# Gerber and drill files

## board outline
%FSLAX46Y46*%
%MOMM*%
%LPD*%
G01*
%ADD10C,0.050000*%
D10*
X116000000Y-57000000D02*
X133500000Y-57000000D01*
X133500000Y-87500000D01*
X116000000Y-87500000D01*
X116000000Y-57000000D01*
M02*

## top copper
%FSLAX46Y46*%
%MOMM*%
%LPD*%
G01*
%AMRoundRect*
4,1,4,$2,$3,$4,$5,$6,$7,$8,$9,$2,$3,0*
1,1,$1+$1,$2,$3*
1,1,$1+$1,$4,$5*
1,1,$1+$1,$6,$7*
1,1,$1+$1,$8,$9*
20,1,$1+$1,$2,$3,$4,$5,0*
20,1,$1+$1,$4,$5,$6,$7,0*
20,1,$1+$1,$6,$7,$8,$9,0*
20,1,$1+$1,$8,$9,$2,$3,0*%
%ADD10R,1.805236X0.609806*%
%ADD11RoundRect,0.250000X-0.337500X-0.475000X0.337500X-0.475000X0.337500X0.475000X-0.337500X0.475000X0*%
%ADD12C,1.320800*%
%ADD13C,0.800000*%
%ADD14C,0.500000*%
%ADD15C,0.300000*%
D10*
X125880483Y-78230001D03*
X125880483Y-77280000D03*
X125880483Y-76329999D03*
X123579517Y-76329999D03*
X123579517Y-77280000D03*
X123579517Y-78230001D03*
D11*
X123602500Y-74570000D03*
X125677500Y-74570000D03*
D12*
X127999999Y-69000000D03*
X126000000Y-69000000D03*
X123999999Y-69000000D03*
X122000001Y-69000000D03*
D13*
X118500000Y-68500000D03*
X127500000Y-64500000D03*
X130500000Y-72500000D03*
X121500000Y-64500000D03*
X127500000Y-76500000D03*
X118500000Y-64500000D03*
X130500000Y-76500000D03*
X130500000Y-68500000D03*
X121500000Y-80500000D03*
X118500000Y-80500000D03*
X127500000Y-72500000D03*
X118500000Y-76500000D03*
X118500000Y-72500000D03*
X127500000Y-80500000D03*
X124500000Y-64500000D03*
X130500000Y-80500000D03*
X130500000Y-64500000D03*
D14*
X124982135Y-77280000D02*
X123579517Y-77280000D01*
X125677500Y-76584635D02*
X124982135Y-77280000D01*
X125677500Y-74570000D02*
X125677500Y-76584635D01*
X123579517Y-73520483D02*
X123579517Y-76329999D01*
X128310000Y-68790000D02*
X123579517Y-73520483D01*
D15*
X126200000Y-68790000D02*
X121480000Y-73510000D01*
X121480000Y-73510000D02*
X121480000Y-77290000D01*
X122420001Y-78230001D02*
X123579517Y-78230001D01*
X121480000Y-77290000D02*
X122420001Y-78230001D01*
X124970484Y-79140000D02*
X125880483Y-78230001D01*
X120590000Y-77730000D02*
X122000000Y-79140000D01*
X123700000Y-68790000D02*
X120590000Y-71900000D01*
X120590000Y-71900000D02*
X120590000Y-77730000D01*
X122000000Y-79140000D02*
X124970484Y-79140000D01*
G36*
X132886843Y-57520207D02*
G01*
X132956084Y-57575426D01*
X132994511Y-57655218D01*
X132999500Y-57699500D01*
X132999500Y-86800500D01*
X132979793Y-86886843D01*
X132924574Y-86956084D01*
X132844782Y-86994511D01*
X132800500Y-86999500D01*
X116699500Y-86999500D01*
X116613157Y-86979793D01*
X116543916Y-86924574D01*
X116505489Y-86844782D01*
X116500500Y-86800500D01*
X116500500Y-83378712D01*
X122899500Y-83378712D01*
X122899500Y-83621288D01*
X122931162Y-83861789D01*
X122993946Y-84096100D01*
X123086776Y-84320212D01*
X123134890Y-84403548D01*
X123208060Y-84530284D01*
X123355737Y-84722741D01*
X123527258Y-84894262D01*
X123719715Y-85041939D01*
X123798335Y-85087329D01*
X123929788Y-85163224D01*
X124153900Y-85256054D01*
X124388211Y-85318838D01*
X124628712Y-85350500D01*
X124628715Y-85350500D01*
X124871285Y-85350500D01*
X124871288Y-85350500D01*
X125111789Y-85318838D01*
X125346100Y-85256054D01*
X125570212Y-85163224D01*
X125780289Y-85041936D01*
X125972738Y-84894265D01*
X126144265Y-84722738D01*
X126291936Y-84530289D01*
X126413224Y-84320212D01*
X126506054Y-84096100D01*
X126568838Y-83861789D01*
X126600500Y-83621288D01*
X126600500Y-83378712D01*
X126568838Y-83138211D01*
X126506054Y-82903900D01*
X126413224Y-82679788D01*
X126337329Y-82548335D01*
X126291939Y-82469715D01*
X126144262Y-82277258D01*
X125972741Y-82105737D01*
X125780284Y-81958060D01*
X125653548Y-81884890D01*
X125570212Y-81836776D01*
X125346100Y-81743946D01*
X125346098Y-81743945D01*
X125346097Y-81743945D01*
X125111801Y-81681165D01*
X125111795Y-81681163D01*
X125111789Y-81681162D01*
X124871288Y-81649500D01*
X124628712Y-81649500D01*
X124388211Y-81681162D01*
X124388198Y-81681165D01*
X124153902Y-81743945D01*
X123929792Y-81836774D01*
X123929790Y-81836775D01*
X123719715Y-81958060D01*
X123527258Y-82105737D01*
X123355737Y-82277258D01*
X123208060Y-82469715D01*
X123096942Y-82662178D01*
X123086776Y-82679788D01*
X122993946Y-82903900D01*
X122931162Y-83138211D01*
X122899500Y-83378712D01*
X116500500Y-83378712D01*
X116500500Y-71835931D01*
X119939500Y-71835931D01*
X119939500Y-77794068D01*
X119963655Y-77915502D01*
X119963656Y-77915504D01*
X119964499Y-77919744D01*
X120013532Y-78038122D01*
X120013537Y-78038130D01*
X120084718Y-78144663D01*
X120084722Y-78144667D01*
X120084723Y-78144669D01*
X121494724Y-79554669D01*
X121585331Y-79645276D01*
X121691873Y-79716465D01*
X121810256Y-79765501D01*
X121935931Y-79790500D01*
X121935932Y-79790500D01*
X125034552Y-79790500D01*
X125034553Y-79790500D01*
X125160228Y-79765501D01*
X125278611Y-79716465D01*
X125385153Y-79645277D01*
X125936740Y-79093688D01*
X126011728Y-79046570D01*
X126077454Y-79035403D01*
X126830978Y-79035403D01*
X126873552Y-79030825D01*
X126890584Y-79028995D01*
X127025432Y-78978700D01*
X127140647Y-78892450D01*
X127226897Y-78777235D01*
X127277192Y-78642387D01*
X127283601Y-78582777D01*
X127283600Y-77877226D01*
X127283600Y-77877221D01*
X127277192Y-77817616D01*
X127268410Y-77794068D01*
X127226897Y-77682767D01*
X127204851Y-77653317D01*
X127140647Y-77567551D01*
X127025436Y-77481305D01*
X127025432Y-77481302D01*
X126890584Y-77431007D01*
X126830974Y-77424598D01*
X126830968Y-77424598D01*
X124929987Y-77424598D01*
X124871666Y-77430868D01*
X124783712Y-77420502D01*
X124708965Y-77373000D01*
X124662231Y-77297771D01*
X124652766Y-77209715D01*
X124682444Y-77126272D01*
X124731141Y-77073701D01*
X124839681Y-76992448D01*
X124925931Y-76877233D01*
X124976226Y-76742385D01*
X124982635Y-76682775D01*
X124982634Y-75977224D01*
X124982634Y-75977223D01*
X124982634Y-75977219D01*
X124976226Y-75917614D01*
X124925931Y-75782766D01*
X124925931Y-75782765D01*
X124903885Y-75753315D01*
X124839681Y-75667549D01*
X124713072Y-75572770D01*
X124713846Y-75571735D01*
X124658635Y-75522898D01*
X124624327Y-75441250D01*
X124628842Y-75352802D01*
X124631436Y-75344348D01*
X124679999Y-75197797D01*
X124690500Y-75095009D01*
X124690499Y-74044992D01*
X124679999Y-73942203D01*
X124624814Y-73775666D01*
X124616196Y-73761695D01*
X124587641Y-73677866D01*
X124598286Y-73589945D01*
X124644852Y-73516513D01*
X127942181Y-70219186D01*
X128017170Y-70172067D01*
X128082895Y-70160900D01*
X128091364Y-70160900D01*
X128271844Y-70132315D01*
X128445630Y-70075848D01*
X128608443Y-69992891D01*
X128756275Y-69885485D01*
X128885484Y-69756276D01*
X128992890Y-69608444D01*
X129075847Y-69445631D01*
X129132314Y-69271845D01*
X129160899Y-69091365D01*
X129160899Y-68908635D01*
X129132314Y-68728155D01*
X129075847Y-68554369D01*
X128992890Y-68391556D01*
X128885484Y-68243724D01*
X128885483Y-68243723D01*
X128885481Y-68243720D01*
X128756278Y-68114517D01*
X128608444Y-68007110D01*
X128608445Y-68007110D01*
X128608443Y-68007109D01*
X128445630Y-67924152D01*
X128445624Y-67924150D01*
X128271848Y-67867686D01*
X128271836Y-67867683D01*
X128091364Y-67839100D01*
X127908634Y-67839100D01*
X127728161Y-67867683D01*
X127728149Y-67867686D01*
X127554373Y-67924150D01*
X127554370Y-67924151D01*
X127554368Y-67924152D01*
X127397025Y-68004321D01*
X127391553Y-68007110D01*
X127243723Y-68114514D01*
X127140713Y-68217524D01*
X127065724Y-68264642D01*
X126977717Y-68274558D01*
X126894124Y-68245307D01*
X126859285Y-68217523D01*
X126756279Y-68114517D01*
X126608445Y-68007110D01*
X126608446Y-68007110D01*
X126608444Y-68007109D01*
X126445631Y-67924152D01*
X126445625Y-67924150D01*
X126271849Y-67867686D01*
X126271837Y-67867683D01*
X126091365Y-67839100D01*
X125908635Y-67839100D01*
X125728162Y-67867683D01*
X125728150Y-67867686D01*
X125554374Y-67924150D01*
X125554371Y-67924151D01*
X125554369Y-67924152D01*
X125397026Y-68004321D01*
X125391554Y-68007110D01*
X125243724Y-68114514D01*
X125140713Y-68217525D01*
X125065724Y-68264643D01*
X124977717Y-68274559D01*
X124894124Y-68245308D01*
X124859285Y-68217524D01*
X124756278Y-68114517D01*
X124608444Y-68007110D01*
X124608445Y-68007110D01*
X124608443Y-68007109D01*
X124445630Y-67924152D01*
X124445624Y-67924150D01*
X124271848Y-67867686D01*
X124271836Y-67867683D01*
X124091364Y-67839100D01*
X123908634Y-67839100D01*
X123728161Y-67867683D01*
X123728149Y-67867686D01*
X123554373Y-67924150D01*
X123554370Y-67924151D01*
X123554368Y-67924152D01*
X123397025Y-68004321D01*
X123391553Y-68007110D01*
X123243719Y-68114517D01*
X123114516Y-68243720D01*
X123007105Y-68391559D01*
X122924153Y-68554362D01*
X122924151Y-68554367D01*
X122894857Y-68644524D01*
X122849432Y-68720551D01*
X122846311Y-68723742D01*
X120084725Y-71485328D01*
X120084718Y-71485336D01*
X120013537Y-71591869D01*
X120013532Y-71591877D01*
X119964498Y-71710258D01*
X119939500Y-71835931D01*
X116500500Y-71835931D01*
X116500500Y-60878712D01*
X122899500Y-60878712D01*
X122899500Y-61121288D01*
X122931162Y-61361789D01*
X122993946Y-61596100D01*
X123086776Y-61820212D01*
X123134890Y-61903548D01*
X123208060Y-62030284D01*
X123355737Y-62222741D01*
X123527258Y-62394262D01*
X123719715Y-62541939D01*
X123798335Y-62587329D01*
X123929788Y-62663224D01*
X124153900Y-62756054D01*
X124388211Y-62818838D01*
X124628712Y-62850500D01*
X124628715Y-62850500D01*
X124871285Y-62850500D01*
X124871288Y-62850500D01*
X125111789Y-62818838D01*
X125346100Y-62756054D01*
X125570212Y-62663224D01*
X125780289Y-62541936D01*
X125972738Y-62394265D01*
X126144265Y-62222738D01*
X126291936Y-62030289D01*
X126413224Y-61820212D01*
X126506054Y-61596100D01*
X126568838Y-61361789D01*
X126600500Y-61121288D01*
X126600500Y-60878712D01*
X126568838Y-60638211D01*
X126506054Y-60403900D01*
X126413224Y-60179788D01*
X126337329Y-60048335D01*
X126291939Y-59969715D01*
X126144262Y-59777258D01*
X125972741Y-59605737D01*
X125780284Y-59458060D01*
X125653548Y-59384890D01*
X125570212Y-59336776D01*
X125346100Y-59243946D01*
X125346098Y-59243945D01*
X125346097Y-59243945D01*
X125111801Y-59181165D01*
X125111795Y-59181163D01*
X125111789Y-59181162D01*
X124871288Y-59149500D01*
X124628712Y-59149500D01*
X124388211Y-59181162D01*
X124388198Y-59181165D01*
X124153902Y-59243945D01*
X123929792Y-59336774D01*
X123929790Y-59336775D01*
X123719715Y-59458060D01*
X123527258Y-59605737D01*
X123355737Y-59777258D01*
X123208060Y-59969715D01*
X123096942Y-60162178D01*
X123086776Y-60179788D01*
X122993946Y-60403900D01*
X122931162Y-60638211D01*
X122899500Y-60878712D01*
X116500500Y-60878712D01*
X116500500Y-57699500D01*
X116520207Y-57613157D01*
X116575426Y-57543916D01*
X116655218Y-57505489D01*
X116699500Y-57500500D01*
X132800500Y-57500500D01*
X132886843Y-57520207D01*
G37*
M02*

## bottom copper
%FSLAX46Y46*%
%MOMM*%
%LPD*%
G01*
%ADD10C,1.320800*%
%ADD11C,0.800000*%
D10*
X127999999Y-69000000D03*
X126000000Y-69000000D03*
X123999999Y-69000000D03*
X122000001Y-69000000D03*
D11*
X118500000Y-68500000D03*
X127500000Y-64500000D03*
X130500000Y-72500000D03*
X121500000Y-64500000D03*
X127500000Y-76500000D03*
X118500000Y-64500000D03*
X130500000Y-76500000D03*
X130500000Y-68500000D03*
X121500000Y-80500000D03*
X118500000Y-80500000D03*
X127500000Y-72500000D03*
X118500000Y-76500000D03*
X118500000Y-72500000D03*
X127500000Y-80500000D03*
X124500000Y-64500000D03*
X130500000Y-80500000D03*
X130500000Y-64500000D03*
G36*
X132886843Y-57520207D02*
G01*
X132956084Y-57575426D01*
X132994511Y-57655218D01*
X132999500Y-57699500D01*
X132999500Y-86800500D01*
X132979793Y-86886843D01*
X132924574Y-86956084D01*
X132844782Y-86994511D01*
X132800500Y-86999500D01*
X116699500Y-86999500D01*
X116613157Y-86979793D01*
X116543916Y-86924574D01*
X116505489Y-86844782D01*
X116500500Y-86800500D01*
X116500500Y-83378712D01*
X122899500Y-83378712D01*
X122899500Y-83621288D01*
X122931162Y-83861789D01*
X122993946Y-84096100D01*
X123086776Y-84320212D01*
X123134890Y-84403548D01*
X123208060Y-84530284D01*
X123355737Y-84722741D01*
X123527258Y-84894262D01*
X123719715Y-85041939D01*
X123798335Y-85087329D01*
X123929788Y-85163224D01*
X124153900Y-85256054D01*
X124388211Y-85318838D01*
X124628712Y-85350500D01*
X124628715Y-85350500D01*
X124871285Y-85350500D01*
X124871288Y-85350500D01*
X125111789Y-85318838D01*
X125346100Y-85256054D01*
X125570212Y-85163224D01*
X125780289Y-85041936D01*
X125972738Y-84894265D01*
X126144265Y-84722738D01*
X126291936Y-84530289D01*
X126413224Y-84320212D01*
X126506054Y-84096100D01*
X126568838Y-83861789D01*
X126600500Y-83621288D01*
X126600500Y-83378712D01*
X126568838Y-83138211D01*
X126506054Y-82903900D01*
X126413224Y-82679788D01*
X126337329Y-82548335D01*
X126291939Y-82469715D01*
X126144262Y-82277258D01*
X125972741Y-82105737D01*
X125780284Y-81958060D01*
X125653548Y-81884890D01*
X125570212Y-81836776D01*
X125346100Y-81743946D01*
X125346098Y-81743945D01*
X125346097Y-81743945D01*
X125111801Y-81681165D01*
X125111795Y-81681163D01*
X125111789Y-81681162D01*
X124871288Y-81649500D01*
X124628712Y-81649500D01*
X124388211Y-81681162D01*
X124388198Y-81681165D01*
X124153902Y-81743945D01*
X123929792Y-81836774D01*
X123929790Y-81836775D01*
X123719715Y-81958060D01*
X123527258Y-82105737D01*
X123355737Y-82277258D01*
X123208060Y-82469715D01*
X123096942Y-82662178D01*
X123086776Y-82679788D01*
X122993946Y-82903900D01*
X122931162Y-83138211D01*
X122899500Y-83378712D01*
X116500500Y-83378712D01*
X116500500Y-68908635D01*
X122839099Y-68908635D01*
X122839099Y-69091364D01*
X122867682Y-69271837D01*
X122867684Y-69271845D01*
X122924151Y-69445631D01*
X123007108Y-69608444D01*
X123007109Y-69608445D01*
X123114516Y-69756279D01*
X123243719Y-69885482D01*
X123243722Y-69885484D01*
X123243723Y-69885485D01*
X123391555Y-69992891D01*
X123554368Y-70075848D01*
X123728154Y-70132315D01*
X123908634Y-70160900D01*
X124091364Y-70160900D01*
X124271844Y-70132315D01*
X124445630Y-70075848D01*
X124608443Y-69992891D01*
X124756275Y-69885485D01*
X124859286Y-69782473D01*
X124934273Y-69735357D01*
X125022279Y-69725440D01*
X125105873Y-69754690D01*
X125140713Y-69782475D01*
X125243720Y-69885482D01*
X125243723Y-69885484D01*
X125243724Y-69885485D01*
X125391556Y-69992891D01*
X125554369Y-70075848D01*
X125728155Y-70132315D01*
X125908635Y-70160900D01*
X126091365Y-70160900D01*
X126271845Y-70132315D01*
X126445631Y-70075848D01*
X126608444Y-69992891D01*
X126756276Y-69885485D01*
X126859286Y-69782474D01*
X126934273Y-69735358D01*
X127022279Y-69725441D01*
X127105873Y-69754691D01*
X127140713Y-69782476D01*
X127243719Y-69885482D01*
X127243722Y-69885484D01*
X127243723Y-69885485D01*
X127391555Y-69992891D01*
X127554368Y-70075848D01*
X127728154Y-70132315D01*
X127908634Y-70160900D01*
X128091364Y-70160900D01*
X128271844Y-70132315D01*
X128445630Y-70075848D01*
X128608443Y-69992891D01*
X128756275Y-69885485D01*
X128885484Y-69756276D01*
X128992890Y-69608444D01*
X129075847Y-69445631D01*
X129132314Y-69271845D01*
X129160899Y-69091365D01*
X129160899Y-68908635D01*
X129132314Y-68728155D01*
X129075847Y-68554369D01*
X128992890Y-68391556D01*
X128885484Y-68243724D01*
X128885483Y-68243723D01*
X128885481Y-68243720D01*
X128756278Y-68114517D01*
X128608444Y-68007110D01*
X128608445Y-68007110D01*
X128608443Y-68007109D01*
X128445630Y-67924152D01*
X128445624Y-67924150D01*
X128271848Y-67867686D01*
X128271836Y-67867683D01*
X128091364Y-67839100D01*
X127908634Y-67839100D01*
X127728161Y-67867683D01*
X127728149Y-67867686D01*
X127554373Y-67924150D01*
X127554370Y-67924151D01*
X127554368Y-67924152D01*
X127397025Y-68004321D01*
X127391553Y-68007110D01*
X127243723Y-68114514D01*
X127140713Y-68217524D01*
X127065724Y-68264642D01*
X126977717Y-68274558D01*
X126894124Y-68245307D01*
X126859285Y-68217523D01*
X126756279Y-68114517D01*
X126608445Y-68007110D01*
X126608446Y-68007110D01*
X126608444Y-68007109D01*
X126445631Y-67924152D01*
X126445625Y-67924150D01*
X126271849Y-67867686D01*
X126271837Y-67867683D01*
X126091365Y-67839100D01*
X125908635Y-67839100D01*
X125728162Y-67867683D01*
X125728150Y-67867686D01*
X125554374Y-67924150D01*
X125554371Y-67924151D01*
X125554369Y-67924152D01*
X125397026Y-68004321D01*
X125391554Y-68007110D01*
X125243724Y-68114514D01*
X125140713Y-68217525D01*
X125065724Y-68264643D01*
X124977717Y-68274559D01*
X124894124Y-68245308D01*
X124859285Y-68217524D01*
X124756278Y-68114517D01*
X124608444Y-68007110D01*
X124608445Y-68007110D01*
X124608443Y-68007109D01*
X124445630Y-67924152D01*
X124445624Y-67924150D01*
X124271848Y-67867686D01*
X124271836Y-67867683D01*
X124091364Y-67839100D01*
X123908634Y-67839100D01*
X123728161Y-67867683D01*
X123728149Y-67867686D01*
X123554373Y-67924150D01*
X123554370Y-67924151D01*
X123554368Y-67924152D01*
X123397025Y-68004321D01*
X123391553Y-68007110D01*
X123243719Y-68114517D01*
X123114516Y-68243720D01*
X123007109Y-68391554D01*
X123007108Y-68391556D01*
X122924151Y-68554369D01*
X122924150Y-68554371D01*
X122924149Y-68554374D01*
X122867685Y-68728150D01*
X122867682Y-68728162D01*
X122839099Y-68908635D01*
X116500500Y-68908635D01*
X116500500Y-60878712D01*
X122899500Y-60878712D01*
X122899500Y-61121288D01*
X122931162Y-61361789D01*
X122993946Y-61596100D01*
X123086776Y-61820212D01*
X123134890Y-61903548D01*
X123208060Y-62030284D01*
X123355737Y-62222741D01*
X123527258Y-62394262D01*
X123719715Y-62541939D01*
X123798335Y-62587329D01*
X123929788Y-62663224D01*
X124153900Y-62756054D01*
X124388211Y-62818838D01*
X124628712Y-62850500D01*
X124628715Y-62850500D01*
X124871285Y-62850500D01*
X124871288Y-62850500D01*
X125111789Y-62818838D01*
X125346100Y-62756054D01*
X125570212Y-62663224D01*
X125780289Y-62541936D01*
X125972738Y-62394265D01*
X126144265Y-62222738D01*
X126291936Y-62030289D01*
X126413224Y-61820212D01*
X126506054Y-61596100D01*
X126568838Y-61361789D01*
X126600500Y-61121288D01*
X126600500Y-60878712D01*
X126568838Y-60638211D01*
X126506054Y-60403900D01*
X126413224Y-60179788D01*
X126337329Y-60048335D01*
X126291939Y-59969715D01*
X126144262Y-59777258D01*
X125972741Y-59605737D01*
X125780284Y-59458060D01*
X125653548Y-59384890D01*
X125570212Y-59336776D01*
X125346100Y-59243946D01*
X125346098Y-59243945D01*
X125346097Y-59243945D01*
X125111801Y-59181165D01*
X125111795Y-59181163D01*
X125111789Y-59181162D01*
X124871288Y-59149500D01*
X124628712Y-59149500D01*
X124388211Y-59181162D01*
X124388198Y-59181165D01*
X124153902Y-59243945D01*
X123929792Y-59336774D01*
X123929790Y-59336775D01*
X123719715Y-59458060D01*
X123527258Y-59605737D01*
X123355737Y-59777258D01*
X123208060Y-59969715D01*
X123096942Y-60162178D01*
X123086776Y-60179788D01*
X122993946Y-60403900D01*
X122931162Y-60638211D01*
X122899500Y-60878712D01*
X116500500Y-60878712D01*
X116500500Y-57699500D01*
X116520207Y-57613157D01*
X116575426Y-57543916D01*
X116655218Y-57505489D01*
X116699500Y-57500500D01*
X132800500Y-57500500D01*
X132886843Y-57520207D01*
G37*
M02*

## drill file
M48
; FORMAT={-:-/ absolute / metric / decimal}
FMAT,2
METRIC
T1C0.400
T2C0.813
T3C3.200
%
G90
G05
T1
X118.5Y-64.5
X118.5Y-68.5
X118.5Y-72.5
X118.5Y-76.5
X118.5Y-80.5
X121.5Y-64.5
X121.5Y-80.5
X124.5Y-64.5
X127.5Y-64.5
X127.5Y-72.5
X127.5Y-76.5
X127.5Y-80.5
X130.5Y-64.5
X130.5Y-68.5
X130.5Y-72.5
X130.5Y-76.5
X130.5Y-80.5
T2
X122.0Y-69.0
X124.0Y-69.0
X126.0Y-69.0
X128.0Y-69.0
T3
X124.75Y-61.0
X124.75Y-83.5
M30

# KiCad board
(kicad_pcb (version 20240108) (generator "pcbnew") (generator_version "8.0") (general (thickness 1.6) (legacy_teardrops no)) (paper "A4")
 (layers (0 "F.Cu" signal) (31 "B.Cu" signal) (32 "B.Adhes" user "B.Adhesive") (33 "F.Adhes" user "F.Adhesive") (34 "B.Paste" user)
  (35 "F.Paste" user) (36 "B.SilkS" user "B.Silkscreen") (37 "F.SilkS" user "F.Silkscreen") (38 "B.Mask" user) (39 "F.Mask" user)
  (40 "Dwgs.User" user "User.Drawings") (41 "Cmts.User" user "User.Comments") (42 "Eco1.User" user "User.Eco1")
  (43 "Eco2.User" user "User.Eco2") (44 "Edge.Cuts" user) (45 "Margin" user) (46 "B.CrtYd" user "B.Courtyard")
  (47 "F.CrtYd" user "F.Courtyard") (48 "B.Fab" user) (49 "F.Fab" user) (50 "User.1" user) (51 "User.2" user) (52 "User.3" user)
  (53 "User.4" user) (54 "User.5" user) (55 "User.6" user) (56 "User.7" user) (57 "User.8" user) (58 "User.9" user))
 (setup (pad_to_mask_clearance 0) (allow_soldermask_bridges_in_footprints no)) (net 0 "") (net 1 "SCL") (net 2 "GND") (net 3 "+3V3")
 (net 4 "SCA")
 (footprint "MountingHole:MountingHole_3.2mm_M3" (layer "F.Cu") (at 124.75 83.5)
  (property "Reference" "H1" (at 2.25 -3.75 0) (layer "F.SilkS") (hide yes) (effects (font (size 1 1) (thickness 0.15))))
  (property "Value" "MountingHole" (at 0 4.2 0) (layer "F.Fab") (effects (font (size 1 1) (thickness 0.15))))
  (pad "" np_thru_hole circle (at 0 0) (size 3.2 3.2) (drill 3.2) (layers "*.Cu" "*.Mask")))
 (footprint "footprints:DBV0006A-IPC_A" (layer "F.Cu") (at 124.73 77.28 180)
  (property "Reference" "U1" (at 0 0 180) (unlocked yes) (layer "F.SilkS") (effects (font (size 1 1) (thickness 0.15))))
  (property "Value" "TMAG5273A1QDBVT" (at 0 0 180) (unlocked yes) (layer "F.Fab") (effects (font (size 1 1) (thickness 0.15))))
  (pad "1" smd rect (at -1.150483 -0.950001 180) (size 1.805236 0.609806) (layers "F.Cu" "F.Paste" "F.Mask") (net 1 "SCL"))
  (pad "2" smd rect (at -1.150483 0 180) (size 1.805236 0.609806) (layers "F.Cu" "F.Paste" "F.Mask") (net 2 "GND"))
  (pad "3" smd rect (at -1.150483 0.950001 180) (size 1.805236 0.609806) (layers "F.Cu" "F.Paste" "F.Mask") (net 2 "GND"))
  (pad "4" smd rect (at 1.150483 0.950001 180) (size 1.805236 0.609806) (layers "F.Cu" "F.Paste" "F.Mask") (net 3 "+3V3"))
  (pad "5" smd rect (at 1.150483 0 180) (size 1.805236 0.609806) (layers "F.Cu" "F.Paste" "F.Mask") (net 2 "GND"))
  (pad "6" smd rect (at 1.150483 -0.950001 180) (size 1.805236 0.609806) (layers "F.Cu" "F.Paste" "F.Mask") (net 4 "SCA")))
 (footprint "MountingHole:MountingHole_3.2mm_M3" (layer "F.Cu") (at 124.75 61)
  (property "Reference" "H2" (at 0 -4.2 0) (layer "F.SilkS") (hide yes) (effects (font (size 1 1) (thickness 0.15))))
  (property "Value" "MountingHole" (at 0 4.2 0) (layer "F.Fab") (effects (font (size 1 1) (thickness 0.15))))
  (pad "" np_thru_hole circle (at 0 0) (size 3.2 3.2) (drill 3.2) (layers "*.Cu" "*.Mask")))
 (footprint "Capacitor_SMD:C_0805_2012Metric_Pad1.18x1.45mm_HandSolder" (layer "F.Cu") (at 124.64 74.57)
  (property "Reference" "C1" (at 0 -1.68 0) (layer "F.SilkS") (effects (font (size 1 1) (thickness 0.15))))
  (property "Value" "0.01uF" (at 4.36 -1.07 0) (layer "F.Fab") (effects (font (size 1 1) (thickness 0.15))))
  (pad "1" smd roundrect (at -1.0375 0) (size 1.175 1.45) (layers "F.Cu" "F.Paste" "F.Mask") (roundrect_rratio 0.212766) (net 3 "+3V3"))
  (pad "2" smd roundrect (at 1.0375 0) (size 1.175 1.45) (layers "F.Cu" "F.Paste" "F.Mask") (roundrect_rratio 0.212766) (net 2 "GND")))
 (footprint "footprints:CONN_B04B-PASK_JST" (layer "B.Cu") (at 127.999999 69 180)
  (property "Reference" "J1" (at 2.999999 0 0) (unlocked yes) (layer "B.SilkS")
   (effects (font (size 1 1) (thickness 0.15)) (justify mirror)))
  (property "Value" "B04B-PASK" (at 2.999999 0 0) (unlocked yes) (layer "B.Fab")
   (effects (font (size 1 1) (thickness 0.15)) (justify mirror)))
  (pad "1" thru_hole circle (at 0 0 180) (size 1.3208 1.3208) (drill 0.8128) (layers "*.Cu" "*.Mask") (remove_unused_layers no)
   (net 3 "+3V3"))
  (pad "2" thru_hole circle (at 1.999999 0 180) (size 1.3208 1.3208) (drill 0.8128) (layers "*.Cu" "*.Mask") (remove_unused_layers no)
   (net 1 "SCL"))
  (pad "3" thru_hole circle (at 4 0 180) (size 1.3208 1.3208) (drill 0.8128) (layers "*.Cu" "*.Mask") (remove_unused_layers no)
   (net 4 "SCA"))
  (pad "4" thru_hole circle (at 5.999998 0 180) (size 1.3208 1.3208) (drill 0.8128) (layers "*.Cu" "*.Mask") (remove_unused_layers no)
   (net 2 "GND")))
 (gr_rect (start 116 57) (end 133.5 87.5) (stroke (width 0.05) (type default)) (fill none) (layer "Edge.Cuts"))
 (segment (start 124.982135 77.28) (end 123.579517 77.28) (width 0.5) (layer "F.Cu") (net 2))
 (segment (start 125.6775 76.584635) (end 124.982135 77.28) (width 0.5) (layer "F.Cu") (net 2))
 (segment (start 125.6775 74.57) (end 125.6775 76.584635) (width 0.5) (layer "F.Cu") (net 2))
 (via (at 118.5 68.5) (size 0.8) (drill 0.4) (layers "F.Cu" "B.Cu") (free yes) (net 2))
 (via (at 127.5 64.5) (size 0.8) (drill 0.4) (layers "F.Cu" "B.Cu") (free yes) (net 2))
 (via (at 130.5 72.5) (size 0.8) (drill 0.4) (layers "F.Cu" "B.Cu") (free yes) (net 2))
 (via (at 121.5 64.5) (size 0.8) (drill 0.4) (layers "F.Cu" "B.Cu") (free yes) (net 2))
 (via (at 127.5 76.5) (size 0.8) (drill 0.4) (layers "F.Cu" "B.Cu") (free yes) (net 2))
 (via (at 118.5 64.5) (size 0.8) (drill 0.4) (layers "F.Cu" "B.Cu") (free yes) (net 2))
 (via (at 130.5 76.5) (size 0.8) (drill 0.4) (layers "F.Cu" "B.Cu") (free yes) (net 2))
 (via (at 130.5 68.5) (size 0.8) (drill 0.4) (layers "F.Cu" "B.Cu") (free yes) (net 2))
 (via (at 121.5 80.5) (size 0.8) (drill 0.4) (layers "F.Cu" "B.Cu") (free yes) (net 2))
 (via (at 118.5 80.5) (size 0.8) (drill 0.4) (layers "F.Cu" "B.Cu") (free yes) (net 2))
 (via (at 127.5 72.5) (size 0.8) (drill 0.4) (layers "F.Cu" "B.Cu") (free yes) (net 2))
 (via (at 118.5 76.5) (size 0.8) (drill 0.4) (layers "F.Cu" "B.Cu") (free yes) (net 2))
 (via (at 118.5 72.5) (size 0.8) (drill 0.4) (layers "F.Cu" "B.Cu") (free yes) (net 2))
 (via (at 127.5 80.5) (size 0.8) (drill 0.4) (layers "F.Cu" "B.Cu") (free yes) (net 2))
 (via (at 124.5 64.5) (size 0.8) (drill 0.4) (layers "F.Cu" "B.Cu") (free yes) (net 2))
 (via (at 130.5 80.5) (size 0.8) (drill 0.4) (layers "F.Cu" "B.Cu") (free yes) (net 2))
 (via (at 130.5 64.5) (size 0.8) (drill 0.4) (layers "F.Cu" "B.Cu") (free yes) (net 2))
 (segment (start 123.579517 73.520483) (end 123.579517 76.329999) (width 0.5) (layer "F.Cu") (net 3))
 (segment (start 128.31 68.79) (end 123.579517 73.520483) (width 0.5) (layer "F.Cu") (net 3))
 (segment (start 126.2 68.79) (end 121.48 73.51) (width 0.3) (layer "F.Cu") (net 1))
 (segment (start 121.48 73.51) (end 121.48 77.29) (width 0.3) (layer "F.Cu") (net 1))
 (segment (start 122.420001 78.230001) (end 123.579517 78.230001) (width 0.3) (layer "F.Cu") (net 1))
 (segment (start 121.48 77.29) (end 122.420001 78.230001) (width 0.3) (layer "F.Cu") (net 1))
 (segment (start 124.970484 79.14) (end 125.880483 78.230001) (width 0.3) (layer "F.Cu") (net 4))
 (segment (start 120.59 77.73) (end 122 79.14) (width 0.3) (layer "F.Cu") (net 4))
 (segment (start 123.7 68.79) (end 120.59 71.9) (width 0.3) (layer "F.Cu") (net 4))
 (segment (start 120.59 71.9) (end 120.59 77.73) (width 0.3) (layer "F.Cu") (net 4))
 (segment (start 122 79.14) (end 124.970484 79.14) (width 0.3) (layer "F.Cu") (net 4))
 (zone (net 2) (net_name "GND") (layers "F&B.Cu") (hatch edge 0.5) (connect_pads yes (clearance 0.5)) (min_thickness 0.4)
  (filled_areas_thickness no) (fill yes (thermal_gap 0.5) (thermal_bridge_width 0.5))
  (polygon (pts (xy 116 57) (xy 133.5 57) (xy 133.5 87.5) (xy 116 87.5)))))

